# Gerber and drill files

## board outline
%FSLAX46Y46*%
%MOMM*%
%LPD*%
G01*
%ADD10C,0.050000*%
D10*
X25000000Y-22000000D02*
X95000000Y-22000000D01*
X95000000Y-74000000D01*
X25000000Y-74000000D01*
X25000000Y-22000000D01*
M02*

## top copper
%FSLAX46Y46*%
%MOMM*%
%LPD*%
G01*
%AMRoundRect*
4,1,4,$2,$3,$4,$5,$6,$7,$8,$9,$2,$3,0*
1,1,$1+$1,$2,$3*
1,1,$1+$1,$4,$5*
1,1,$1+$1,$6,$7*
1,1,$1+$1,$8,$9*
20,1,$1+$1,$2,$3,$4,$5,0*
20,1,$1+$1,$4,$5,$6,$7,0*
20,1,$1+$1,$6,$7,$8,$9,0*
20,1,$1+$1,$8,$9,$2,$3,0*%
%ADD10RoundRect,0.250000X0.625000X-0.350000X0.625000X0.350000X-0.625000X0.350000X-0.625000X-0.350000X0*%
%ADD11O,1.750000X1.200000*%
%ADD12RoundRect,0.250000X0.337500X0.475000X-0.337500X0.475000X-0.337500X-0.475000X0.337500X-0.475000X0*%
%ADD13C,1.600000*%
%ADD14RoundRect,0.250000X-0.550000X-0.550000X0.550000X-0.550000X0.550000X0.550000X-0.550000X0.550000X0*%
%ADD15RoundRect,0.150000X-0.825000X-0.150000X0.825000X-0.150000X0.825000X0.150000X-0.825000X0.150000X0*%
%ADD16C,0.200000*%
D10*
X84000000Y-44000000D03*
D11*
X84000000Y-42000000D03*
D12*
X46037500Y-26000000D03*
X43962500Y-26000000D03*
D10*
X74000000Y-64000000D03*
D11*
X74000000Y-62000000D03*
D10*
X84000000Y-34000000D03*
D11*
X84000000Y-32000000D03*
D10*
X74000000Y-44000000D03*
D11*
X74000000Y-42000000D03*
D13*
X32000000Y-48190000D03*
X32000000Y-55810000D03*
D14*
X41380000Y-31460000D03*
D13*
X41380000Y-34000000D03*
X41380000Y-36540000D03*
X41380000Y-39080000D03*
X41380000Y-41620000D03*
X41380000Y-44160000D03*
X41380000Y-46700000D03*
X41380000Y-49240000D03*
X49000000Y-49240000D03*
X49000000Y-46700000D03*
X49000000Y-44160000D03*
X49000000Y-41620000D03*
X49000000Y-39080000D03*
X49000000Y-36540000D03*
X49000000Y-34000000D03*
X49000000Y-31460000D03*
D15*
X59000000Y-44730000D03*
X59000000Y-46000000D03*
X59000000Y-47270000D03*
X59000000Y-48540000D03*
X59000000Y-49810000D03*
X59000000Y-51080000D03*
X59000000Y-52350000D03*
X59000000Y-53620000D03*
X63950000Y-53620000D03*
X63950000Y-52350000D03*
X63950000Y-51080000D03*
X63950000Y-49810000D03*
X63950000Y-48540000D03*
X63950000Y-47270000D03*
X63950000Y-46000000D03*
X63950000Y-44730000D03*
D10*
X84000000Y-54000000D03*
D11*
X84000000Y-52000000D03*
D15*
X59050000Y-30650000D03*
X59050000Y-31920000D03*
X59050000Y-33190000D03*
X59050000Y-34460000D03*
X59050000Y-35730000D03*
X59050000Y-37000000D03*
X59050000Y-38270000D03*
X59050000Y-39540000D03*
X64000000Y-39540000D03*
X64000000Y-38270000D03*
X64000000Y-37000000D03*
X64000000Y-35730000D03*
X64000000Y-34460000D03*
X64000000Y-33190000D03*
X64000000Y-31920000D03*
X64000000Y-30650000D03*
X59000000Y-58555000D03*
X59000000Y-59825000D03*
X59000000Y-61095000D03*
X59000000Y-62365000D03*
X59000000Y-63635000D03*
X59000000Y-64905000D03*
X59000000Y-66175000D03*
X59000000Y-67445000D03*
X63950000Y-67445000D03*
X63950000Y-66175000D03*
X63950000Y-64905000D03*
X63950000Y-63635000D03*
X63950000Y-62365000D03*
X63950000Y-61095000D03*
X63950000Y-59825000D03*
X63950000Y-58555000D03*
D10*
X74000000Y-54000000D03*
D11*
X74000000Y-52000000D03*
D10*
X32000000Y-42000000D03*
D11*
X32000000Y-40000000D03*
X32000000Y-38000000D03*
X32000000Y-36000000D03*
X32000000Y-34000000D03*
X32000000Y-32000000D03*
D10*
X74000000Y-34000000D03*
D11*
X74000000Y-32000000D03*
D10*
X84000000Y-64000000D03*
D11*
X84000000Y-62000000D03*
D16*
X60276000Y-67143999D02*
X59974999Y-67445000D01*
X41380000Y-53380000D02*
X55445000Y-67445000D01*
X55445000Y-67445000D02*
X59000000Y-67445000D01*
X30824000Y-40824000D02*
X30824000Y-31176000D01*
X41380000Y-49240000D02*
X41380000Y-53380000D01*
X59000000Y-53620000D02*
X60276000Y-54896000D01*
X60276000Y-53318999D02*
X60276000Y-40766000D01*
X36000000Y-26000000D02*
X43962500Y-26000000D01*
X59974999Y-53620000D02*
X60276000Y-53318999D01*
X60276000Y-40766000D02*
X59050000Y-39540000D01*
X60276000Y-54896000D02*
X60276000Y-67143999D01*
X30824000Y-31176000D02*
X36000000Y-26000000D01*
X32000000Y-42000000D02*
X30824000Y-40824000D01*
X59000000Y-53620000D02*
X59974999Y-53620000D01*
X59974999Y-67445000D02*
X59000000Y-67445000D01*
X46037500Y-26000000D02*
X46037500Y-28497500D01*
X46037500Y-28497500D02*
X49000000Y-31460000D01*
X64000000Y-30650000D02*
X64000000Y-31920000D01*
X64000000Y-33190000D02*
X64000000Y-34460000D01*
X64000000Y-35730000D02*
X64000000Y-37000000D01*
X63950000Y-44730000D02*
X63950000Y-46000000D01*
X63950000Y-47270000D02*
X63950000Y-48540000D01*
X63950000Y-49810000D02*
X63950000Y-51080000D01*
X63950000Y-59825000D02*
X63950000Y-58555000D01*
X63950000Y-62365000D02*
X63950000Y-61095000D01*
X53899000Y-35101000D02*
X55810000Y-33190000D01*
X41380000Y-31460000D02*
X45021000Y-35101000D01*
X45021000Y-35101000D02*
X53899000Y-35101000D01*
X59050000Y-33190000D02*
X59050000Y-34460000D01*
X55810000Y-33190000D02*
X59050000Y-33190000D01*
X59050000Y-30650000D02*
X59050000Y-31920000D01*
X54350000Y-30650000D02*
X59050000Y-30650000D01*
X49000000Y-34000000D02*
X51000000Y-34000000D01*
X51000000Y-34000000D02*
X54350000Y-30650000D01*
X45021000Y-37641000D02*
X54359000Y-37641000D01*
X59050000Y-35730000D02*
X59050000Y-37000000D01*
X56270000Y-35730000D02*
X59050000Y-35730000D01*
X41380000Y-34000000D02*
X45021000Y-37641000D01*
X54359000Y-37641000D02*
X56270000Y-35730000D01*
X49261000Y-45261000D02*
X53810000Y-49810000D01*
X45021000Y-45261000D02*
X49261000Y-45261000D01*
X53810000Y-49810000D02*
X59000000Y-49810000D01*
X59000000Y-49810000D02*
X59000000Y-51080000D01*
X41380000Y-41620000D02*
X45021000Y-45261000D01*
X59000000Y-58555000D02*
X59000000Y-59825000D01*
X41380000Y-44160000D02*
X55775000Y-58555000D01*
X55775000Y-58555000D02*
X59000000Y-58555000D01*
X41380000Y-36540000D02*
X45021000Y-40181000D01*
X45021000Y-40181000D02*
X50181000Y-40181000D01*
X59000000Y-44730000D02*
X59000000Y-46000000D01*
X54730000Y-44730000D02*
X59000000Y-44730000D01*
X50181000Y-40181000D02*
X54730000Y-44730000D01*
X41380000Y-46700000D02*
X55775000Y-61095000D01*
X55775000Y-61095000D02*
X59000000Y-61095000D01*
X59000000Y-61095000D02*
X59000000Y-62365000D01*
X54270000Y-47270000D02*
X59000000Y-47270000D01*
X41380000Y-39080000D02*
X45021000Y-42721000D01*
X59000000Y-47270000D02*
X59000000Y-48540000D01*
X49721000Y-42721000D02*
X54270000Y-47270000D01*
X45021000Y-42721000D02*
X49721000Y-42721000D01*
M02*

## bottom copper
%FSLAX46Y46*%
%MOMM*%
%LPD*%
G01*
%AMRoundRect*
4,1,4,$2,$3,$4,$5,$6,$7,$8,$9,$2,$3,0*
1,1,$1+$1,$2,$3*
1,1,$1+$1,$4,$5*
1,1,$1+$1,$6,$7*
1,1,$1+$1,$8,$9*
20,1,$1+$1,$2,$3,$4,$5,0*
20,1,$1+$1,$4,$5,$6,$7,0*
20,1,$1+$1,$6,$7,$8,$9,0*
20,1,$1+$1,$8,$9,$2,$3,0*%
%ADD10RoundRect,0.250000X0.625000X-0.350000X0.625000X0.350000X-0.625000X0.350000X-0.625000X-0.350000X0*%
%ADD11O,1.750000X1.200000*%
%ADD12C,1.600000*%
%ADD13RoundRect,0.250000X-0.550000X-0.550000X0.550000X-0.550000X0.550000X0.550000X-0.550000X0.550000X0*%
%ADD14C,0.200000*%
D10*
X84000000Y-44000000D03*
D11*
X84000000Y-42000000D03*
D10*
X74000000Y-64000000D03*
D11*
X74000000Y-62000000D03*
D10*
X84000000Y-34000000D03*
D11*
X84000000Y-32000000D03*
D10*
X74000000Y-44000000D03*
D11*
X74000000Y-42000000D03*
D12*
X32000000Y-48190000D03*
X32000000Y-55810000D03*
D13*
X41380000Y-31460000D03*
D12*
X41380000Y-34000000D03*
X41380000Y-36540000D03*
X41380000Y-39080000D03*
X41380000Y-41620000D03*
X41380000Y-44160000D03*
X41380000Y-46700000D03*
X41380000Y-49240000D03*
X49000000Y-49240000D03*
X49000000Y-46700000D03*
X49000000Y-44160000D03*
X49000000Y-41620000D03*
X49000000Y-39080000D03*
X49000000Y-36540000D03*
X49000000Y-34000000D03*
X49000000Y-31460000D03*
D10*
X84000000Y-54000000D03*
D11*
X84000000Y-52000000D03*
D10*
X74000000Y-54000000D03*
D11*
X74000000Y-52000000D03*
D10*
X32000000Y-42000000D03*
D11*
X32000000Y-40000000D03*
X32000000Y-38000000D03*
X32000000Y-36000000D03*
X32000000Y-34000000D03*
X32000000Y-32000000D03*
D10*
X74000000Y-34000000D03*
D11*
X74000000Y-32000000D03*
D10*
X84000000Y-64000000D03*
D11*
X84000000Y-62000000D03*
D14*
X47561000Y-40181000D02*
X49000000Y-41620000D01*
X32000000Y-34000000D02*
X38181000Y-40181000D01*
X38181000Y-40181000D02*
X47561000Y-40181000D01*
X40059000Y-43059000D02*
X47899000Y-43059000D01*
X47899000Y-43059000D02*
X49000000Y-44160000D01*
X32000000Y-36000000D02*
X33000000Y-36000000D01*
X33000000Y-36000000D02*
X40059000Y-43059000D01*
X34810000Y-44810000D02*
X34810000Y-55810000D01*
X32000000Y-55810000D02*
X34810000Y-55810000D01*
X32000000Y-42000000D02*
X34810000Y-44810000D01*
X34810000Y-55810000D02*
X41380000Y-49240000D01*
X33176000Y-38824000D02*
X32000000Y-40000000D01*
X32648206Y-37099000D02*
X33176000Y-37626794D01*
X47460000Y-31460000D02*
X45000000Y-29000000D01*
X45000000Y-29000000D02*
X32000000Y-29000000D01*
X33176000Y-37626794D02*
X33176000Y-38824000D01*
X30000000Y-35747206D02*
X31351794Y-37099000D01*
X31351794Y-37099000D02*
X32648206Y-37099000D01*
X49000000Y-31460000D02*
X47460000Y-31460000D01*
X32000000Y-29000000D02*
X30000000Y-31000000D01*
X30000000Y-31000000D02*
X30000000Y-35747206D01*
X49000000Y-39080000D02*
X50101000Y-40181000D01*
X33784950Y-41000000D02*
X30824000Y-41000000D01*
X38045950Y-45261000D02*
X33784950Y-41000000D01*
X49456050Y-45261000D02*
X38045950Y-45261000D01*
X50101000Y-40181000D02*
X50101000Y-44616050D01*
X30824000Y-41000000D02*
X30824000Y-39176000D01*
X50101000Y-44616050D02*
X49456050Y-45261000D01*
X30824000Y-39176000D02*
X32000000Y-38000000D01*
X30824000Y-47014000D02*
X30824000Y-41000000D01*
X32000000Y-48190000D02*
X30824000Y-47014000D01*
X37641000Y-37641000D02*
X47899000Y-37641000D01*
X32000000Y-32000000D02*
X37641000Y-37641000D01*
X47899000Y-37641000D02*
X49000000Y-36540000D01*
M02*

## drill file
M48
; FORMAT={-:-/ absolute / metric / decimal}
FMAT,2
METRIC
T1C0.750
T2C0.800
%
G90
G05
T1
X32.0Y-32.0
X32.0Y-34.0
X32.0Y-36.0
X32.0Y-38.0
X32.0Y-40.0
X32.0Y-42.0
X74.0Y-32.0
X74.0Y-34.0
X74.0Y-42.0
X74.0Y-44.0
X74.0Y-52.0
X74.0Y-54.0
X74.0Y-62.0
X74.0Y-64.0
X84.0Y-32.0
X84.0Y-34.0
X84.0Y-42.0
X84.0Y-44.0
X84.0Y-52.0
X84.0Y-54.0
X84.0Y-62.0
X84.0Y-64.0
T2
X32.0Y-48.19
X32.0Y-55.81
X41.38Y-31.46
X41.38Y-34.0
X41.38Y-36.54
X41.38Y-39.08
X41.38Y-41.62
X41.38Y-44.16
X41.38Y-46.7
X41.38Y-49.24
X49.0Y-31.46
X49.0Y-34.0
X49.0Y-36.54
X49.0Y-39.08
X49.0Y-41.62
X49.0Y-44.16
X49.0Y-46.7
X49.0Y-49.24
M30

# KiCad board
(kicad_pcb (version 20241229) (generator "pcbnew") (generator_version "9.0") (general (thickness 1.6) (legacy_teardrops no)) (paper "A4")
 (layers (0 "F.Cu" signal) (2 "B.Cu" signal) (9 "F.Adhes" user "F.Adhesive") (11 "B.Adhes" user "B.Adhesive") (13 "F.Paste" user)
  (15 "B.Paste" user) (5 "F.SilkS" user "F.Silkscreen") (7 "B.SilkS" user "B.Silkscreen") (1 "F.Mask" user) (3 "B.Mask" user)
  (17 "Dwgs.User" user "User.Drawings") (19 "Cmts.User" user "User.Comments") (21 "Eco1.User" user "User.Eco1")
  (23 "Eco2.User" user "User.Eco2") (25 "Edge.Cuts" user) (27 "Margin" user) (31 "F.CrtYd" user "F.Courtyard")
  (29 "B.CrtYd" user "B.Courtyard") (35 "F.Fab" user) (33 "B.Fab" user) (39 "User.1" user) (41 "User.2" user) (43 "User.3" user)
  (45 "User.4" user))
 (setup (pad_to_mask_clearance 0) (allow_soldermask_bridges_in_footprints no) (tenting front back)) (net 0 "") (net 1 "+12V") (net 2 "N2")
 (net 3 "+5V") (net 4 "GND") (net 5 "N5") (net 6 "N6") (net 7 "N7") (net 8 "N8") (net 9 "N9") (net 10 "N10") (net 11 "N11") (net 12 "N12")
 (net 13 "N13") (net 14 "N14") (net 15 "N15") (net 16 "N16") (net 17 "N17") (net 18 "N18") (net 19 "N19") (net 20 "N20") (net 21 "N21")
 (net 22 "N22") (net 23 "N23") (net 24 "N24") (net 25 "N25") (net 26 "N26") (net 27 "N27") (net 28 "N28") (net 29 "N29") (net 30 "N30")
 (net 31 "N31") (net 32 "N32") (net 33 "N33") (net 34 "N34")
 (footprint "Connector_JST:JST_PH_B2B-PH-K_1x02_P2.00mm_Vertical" (layer "F.Cu") (at 84 44 90)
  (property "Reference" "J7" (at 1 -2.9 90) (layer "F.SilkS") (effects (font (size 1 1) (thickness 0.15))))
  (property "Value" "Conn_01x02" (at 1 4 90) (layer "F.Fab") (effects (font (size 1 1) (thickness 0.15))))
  (pad "1" thru_hole roundrect (at 0 0 90) (size 1.2 1.75) (drill 0.75) (layers "*.Cu" "*.Mask") (remove_unused_layers no)
   (roundrect_rratio 0.208333) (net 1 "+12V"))
  (pad "2" thru_hole oval (at 2 0 90) (size 1.2 1.75) (drill 0.75) (layers "*.Cu" "*.Mask") (remove_unused_layers no) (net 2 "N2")))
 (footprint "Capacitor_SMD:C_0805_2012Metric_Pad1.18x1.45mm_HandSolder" (layer "F.Cu") (at 45 26 180)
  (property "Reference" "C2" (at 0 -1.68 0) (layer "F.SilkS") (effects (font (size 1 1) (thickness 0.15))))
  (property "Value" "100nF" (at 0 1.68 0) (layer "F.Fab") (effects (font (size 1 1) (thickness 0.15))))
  (pad "1" smd roundrect (at -1.0375 0 180) (size 1.175 1.45) (layers "F.Cu" "F.Mask" "F.Paste") (roundrect_rratio 0.212766) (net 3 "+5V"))
  (pad "2" smd roundrect (at 1.0375 0 180) (size 1.175 1.45) (layers "F.Cu" "F.Mask" "F.Paste") (roundrect_rratio 0.212766) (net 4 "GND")))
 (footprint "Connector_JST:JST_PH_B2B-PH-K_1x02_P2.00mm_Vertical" (layer "F.Cu") (at 74 64 90)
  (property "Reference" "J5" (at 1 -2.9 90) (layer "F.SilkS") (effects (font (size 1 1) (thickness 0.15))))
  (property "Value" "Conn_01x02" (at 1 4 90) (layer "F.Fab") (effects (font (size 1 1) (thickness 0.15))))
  (pad "1" thru_hole roundrect (at 0 0 90) (size 1.2 1.75) (drill 0.75) (layers "*.Cu" "*.Mask") (remove_unused_layers no)
   (roundrect_rratio 0.208333) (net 1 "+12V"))
  (pad "2" thru_hole oval (at 2 0 90) (size 1.2 1.75) (drill 0.75) (layers "*.Cu" "*.Mask") (remove_unused_layers no) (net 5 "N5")))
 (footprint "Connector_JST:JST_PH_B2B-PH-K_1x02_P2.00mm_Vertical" (layer "F.Cu") (at 84 34 90)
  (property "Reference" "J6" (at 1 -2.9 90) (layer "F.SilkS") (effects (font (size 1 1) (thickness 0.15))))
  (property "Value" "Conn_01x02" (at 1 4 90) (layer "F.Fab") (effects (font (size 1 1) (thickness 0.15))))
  (pad "1" thru_hole roundrect (at 0 0 90) (size 1.2 1.75) (drill 0.75) (layers "*.Cu" "*.Mask") (remove_unused_layers no)
   (roundrect_rratio 0.208333) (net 1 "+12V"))
  (pad "2" thru_hole oval (at 2 0 90) (size 1.2 1.75) (drill 0.75) (layers "*.Cu" "*.Mask") (remove_unused_layers no) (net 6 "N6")))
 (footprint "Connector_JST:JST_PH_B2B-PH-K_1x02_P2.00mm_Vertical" (layer "F.Cu") (at 74 44 90)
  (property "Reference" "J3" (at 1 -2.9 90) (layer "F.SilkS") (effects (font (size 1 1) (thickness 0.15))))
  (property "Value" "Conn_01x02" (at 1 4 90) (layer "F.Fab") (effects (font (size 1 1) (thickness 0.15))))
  (pad "1" thru_hole roundrect (at 0 0 90) (size 1.2 1.75) (drill 0.75) (layers "*.Cu" "*.Mask") (remove_unused_layers no)
   (roundrect_rratio 0.208333) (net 1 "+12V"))
  (pad "2" thru_hole oval (at 2 0 90) (size 1.2 1.75) (drill 0.75) (layers "*.Cu" "*.Mask") (remove_unused_layers no) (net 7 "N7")))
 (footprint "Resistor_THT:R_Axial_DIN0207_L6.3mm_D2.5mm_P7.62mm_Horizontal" (layer "F.Cu") (at 32 48.19 -90)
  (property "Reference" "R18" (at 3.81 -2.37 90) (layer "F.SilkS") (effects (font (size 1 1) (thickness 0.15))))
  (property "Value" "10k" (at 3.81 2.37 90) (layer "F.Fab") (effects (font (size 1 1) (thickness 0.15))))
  (pad "1" thru_hole circle (at 0 0 270) (size 1.6 1.6) (drill 0.8) (layers "*.Cu" "*.Mask") (remove_unused_layers no) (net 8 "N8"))
  (pad "2" thru_hole circle (at 7.62 0 270) (size 1.6 1.6) (drill 0.8) (layers "*.Cu" "*.Mask") (remove_unused_layers no) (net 4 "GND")))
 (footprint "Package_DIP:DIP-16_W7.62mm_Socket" (layer "F.Cu") (at 41.38 31.46)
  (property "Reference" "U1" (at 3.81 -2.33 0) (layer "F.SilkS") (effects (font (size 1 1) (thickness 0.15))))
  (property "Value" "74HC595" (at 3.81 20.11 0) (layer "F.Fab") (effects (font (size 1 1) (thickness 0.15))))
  (pad "1" thru_hole roundrect (at 0 0) (size 1.6 1.6) (drill 0.8) (layers "*.Cu" "*.Mask") (remove_unused_layers no)
   (roundrect_rratio 0.15625) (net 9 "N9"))
  (pad "2" thru_hole circle (at 0 2.54) (size 1.6 1.6) (drill 0.8) (layers "*.Cu" "*.Mask") (remove_unused_layers no) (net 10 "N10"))
  (pad "3" thru_hole circle (at 0 5.08) (size 1.6 1.6) (drill 0.8) (layers "*.Cu" "*.Mask") (remove_unused_layers no) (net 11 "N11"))
  (pad "4" thru_hole circle (at 0 7.62) (size 1.6 1.6) (drill 0.8) (layers "*.Cu" "*.Mask") (remove_unused_layers no) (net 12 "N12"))
  (pad "5" thru_hole circle (at 0 10.16) (size 1.6 1.6) (drill 0.8) (layers "*.Cu" "*.Mask") (remove_unused_layers no) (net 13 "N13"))
  (pad "6" thru_hole circle (at 0 12.7) (size 1.6 1.6) (drill 0.8) (layers "*.Cu" "*.Mask") (remove_unused_layers no) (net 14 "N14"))
  (pad "7" thru_hole circle (at 0 15.24) (size 1.6 1.6) (drill 0.8) (layers "*.Cu" "*.Mask") (remove_unused_layers no) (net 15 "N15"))
  (pad "8" thru_hole circle (at 0 17.78) (size 1.6 1.6) (drill 0.8) (layers "*.Cu" "*.Mask") (remove_unused_layers no) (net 4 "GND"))
  (pad "9" thru_hole circle (at 7.62 17.78) (size 1.6 1.6) (drill 0.8) (layers "*.Cu" "*.Mask") (remove_unused_layers no) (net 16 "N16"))
  (pad "10" thru_hole circle (at 7.62 15.24) (size 1.6 1.6) (drill 0.8) (layers "*.Cu" "*.Mask") (remove_unused_layers no) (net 3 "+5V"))
  (pad "11" thru_hole circle (at 7.62 12.7) (size 1.6 1.6) (drill 0.8) (layers "*.Cu" "*.Mask") (remove_unused_layers no) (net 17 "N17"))
  (pad "12" thru_hole circle (at 7.62 10.16) (size 1.6 1.6) (drill 0.8) (layers "*.Cu" "*.Mask") (remove_unused_layers no) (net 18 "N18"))
  (pad "13" thru_hole circle (at 7.62 7.62) (size 1.6 1.6) (drill 0.8) (layers "*.Cu" "*.Mask") (remove_unused_layers no) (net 8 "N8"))
  (pad "14" thru_hole circle (at 7.62 5.08) (size 1.6 1.6) (drill 0.8) (layers "*.Cu" "*.Mask") (remove_unused_layers no) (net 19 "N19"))
  (pad "15" thru_hole circle (at 7.62 2.54) (size 1.6 1.6) (drill 0.8) (layers "*.Cu" "*.Mask") (remove_unused_layers no) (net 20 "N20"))
  (pad "16" thru_hole circle (at 7.62 0) (size 1.6 1.6) (drill 0.8) (layers "*.Cu" "*.Mask") (remove_unused_layers no) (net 3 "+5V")))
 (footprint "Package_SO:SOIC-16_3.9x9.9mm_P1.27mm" (layer "F.Cu") (at 61.475 49.175)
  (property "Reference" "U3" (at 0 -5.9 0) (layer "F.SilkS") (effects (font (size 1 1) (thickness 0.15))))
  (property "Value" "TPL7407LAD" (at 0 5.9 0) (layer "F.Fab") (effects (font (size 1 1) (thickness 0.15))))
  (pad "1" smd roundrect (at -2.475 -4.445) (size 1.95 0.6) (layers "F.Cu" "F.Mask" "F.Paste") (roundrect_rratio 0.25) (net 11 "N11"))
  (pad "2" smd roundrect (at -2.475 -3.175) (size 1.95 0.6) (layers "F.Cu" "F.Mask" "F.Paste") (roundrect_rratio 0.25) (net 11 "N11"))
  (pad "3" smd roundrect (at -2.475 -1.905) (size 1.95 0.6) (layers "F.Cu" "F.Mask" "F.Paste") (roundrect_rratio 0.25) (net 12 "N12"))
  (pad "4" smd roundrect (at -2.475 -0.635) (size 1.95 0.6) (layers "F.Cu" "F.Mask" "F.Paste") (roundrect_rratio 0.25) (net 12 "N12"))
  (pad "5" smd roundrect (at -2.475 0.635) (size 1.95 0.6) (layers "F.Cu" "F.Mask" "F.Paste") (roundrect_rratio 0.25) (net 13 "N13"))
  (pad "6" smd roundrect (at -2.475 1.905) (size 1.95 0.6) (layers "F.Cu" "F.Mask" "F.Paste") (roundrect_rratio 0.25) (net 13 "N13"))
  (pad "7" smd roundrect (at -2.475 3.175) (size 1.95 0.6) (layers "F.Cu" "F.Mask" "F.Paste") (roundrect_rratio 0.25) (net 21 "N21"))
  (pad "8" smd roundrect (at -2.475 4.445) (size 1.95 0.6) (layers "F.Cu" "F.Mask" "F.Paste") (roundrect_rratio 0.25) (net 4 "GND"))
  (pad "9" smd roundrect (at 2.475 4.445) (size 1.95 0.6) (layers "F.Cu" "F.Mask" "F.Paste") (roundrect_rratio 0.25) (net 1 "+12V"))
  (pad "10" smd roundrect (at 2.475 3.175) (size 1.95 0.6) (layers "F.Cu" "F.Mask" "F.Paste") (roundrect_rratio 0.25) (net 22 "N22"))
  (pad "11" smd roundrect (at 2.475 1.905) (size 1.95 0.6) (layers "F.Cu" "F.Mask" "F.Paste") (roundrect_rratio 0.25) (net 2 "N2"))
  (pad "12" smd roundrect (at 2.475 0.635) (size 1.95 0.6) (layers "F.Cu" "F.Mask" "F.Paste") (roundrect_rratio 0.25) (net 2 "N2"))
  (pad "13" smd roundrect (at 2.475 -0.635) (size 1.95 0.6) (layers "F.Cu" "F.Mask" "F.Paste") (roundrect_rratio 0.25) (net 6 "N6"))
  (pad "14" smd roundrect (at 2.475 -1.905) (size 1.95 0.6) (layers "F.Cu" "F.Mask" "F.Paste") (roundrect_rratio 0.25) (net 6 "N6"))
  (pad "15" smd roundrect (at 2.475 -3.175) (size 1.95 0.6) (layers "F.Cu" "F.Mask" "F.Paste") (roundrect_rratio 0.25) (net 5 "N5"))
  (pad "16" smd roundrect (at 2.475 -4.445) (size 1.95 0.6) (layers "F.Cu" "F.Mask" "F.Paste") (roundrect_rratio 0.25) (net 5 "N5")))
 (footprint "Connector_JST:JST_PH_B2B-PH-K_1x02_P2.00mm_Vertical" (layer "F.Cu") (at 84 54 90)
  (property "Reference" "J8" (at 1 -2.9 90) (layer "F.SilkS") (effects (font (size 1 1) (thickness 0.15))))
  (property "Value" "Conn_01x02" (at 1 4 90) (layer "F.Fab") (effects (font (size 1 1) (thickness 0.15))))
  (pad "1" thru_hole roundrect (at 0 0 90) (size 1.2 1.75) (drill 0.75) (layers "*.Cu" "*.Mask") (remove_unused_layers no)
   (roundrect_rratio 0.208333) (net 1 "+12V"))
  (pad "2" thru_hole oval (at 2 0 90) (size 1.2 1.75) (drill 0.75) (layers "*.Cu" "*.Mask") (remove_unused_layers no) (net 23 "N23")))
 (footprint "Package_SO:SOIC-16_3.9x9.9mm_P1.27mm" (layer "F.Cu") (at 61.525 35.095)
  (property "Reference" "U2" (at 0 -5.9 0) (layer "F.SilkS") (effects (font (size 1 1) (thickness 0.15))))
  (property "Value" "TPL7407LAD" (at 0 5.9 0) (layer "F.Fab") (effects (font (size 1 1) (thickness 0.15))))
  (pad "1" smd roundrect (at -2.475 -4.445) (size 1.95 0.6) (layers "F.Cu" "F.Mask" "F.Paste") (roundrect_rratio 0.25) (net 20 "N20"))
  (pad "2" smd roundrect (at -2.475 -3.175) (size 1.95 0.6) (layers "F.Cu" "F.Mask" "F.Paste") (roundrect_rratio 0.25) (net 20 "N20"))
  (pad "3" smd roundrect (at -2.475 -1.905) (size 1.95 0.6) (layers "F.Cu" "F.Mask" "F.Paste") (roundrect_rratio 0.25) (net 9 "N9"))
  (pad "4" smd roundrect (at -2.475 -0.635) (size 1.95 0.6) (layers "F.Cu" "F.Mask" "F.Paste") (roundrect_rratio 0.25) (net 9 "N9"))
  (pad "5" smd roundrect (at -2.475 0.635) (size 1.95 0.6) (layers "F.Cu" "F.Mask" "F.Paste") (roundrect_rratio 0.25) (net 10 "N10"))
  (pad "6" smd roundrect (at -2.475 1.905) (size 1.95 0.6) (layers "F.Cu" "F.Mask" "F.Paste") (roundrect_rratio 0.25) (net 10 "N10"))
  (pad "7" smd roundrect (at -2.475 3.175) (size 1.95 0.6) (layers "F.Cu" "F.Mask" "F.Paste") (roundrect_rratio 0.25) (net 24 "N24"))
  (pad "8" smd roundrect (at -2.475 4.445) (size 1.95 0.6) (layers "F.Cu" "F.Mask" "F.Paste") (roundrect_rratio 0.25) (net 4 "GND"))
  (pad "9" smd roundrect (at 2.475 4.445) (size 1.95 0.6) (layers "F.Cu" "F.Mask" "F.Paste") (roundrect_rratio 0.25) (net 1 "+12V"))
  (pad "10" smd roundrect (at 2.475 3.175) (size 1.95 0.6) (layers "F.Cu" "F.Mask" "F.Paste") (roundrect_rratio 0.25) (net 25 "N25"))
  (pad "11" smd roundrect (at 2.475 1.905) (size 1.95 0.6) (layers "F.Cu" "F.Mask" "F.Paste") (roundrect_rratio 0.25) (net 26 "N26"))
  (pad "12" smd roundrect (at 2.475 0.635) (size 1.95 0.6) (layers "F.Cu" "F.Mask" "F.Paste") (roundrect_rratio 0.25) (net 26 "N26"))
  (pad "13" smd roundrect (at 2.475 -0.635) (size 1.95 0.6) (layers "F.Cu" "F.Mask" "F.Paste") (roundrect_rratio 0.25) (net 7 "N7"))
  (pad "14" smd roundrect (at 2.475 -1.905) (size 1.95 0.6) (layers "F.Cu" "F.Mask" "F.Paste") (roundrect_rratio 0.25) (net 7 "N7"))
  (pad "15" smd roundrect (at 2.475 -3.175) (size 1.95 0.6) (layers "F.Cu" "F.Mask" "F.Paste") (roundrect_rratio 0.25) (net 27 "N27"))
  (pad "16" smd roundrect (at 2.475 -4.445) (size 1.95 0.6) (layers "F.Cu" "F.Mask" "F.Paste") (roundrect_rratio 0.25) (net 27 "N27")))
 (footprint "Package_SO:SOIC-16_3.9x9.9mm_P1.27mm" (layer "F.Cu") (at 61.475 63)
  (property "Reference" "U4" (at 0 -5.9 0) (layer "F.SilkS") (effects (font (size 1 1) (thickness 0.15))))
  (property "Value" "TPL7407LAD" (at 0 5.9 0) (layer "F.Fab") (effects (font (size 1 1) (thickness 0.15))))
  (pad "1" smd roundrect (at -2.475 -4.445) (size 1.95 0.6) (layers "F.Cu" "F.Mask" "F.Paste") (roundrect_rratio 0.25) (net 14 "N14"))
  (pad "2" smd roundrect (at -2.475 -3.175) (size 1.95 0.6) (layers "F.Cu" "F.Mask" "F.Paste") (roundrect_rratio 0.25) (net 14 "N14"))
  (pad "3" smd roundrect (at -2.475 -1.905) (size 1.95 0.6) (layers "F.Cu" "F.Mask" "F.Paste") (roundrect_rratio 0.25) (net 15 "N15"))
  (pad "4" smd roundrect (at -2.475 -0.635) (size 1.95 0.6) (layers "F.Cu" "F.Mask" "F.Paste") (roundrect_rratio 0.25) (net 15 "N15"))
  (pad "5" smd roundrect (at -2.475 0.635) (size 1.95 0.6) (layers "F.Cu" "F.Mask" "F.Paste") (roundrect_rratio 0.25) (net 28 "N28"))
  (pad "6" smd roundrect (at -2.475 1.905) (size 1.95 0.6) (layers "F.Cu" "F.Mask" "F.Paste") (roundrect_rratio 0.25) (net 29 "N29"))
  (pad "7" smd roundrect (at -2.475 3.175) (size 1.95 0.6) (layers "F.Cu" "F.Mask" "F.Paste") (roundrect_rratio 0.25) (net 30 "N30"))
  (pad "8" smd roundrect (at -2.475 4.445) (size 1.95 0.6) (layers "F.Cu" "F.Mask" "F.Paste") (roundrect_rratio 0.25) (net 4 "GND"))
  (pad "9" smd roundrect (at 2.475 4.445) (size 1.95 0.6) (layers "F.Cu" "F.Mask" "F.Paste") (roundrect_rratio 0.25) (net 1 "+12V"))
  (pad "10" smd roundrect (at 2.475 3.175) (size 1.95 0.6) (layers "F.Cu" "F.Mask" "F.Paste") (roundrect_rratio 0.25) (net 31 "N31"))
  (pad "11" smd roundrect (at 2.475 1.905) (size 1.95 0.6) (layers "F.Cu" "F.Mask" "F.Paste") (roundrect_rratio 0.25) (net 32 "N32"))
  (pad "12" smd roundrect (at 2.475 0.635) (size 1.95 0.6) (layers "F.Cu" "F.Mask" "F.Paste") (roundrect_rratio 0.25) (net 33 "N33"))
  (pad "13" smd roundrect (at 2.475 -0.635) (size 1.95 0.6) (layers "F.Cu" "F.Mask" "F.Paste") (roundrect_rratio 0.25) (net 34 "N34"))
  (pad "14" smd roundrect (at 2.475 -1.905) (size 1.95 0.6) (layers "F.Cu" "F.Mask" "F.Paste") (roundrect_rratio 0.25) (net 34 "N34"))
  (pad "15" smd roundrect (at 2.475 -3.175) (size 1.95 0.6) (layers "F.Cu" "F.Mask" "F.Paste") (roundrect_rratio 0.25) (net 23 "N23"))
  (pad "16" smd roundrect (at 2.475 -4.445) (size 1.95 0.6) (layers "F.Cu" "F.Mask" "F.Paste") (roundrect_rratio 0.25) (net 23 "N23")))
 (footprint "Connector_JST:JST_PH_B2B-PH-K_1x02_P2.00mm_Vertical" (layer "F.Cu") (at 74 54 90)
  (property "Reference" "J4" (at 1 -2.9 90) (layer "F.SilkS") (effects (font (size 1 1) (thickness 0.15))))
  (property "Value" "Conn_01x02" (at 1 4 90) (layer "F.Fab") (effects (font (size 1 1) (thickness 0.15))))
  (pad "1" thru_hole roundrect (at 0 0 90) (size 1.2 1.75) (drill 0.75) (layers "*.Cu" "*.Mask") (remove_unused_layers no)
   (roundrect_rratio 0.208333) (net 1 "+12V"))
  (pad "2" thru_hole oval (at 2 0 90) (size 1.2 1.75) (drill 0.75) (layers "*.Cu" "*.Mask") (remove_unused_layers no) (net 26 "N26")))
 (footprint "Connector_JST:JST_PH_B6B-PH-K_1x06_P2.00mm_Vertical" (layer "F.Cu") (at 32 42 90)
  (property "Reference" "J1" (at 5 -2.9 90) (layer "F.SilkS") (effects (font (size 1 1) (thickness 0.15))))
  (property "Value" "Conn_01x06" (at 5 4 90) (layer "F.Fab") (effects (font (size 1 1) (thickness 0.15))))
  (pad "1" thru_hole roundrect (at 0 0 90) (size 1.2 1.75) (drill 0.75) (layers "*.Cu" "*.Mask") (remove_unused_layers no)
   (roundrect_rratio 0.208333) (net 4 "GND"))
  (pad "2" thru_hole oval (at 2 0 90) (size 1.2 1.75) (drill 0.75) (layers "*.Cu" "*.Mask") (remove_unused_layers no) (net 3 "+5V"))
  (pad "3" thru_hole oval (at 4 0 90) (size 1.2 1.75) (drill 0.75) (layers "*.Cu" "*.Mask") (remove_unused_layers no) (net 8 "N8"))
  (pad "4" thru_hole oval (at 6 0 90) (size 1.2 1.75) (drill 0.75) (layers "*.Cu" "*.Mask") (remove_unused_layers no) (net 17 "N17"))
  (pad "5" thru_hole oval (at 8 0 90) (size 1.2 1.75) (drill 0.75) (layers "*.Cu" "*.Mask") (remove_unused_layers no) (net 18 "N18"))
  (pad "6" thru_hole oval (at 10 0 90) (size 1.2 1.75) (drill 0.75) (layers "*.Cu" "*.Mask") (remove_unused_layers no) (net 19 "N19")))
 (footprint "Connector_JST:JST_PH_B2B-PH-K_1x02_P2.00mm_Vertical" (layer "F.Cu") (at 74 34 90)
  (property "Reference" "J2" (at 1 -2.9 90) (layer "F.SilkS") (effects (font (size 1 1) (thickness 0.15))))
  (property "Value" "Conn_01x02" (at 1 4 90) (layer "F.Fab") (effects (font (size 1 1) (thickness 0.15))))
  (pad "1" thru_hole roundrect (at 0 0 90) (size 1.2 1.75) (drill 0.75) (layers "*.Cu" "*.Mask") (remove_unused_layers no)
   (roundrect_rratio 0.208333) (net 1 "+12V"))
  (pad "2" thru_hole oval (at 2 0 90) (size 1.2 1.75) (drill 0.75) (layers "*.Cu" "*.Mask") (remove_unused_layers no) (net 27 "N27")))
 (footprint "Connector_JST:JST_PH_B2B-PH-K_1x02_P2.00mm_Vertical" (layer "F.Cu") (at 84 64 90)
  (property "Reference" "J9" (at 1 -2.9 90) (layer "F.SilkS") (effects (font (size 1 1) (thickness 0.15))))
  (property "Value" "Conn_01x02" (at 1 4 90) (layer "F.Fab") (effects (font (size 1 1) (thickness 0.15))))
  (pad "1" thru_hole roundrect (at 0 0 90) (size 1.2 1.75) (drill 0.75) (layers "*.Cu" "*.Mask") (remove_unused_layers no)
   (roundrect_rratio 0.208333) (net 1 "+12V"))
  (pad "2" thru_hole oval (at 2 0 90) (size 1.2 1.75) (drill 0.75) (layers "*.Cu" "*.Mask") (remove_unused_layers no) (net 34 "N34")))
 (gr_rect (start 25 22) (end 95 74) (stroke (width 0.05) (type default)) (fill no) (layer "Edge.Cuts"))
 (segment (start 47.561 40.181) (end 49 41.62) (width 0.2) (layer "B.Cu") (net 18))
 (segment (start 32 34) (end 38.181 40.181) (width 0.2) (layer "B.Cu") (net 18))
 (segment (start 38.181 40.181) (end 47.561 40.181) (width 0.2) (layer "B.Cu") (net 18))
 (segment (start 40.059 43.059) (end 47.899 43.059) (width 0.2) (layer "B.Cu") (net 17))
 (segment (start 47.899 43.059) (end 49 44.16) (width 0.2) (layer "B.Cu") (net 17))
 (segment (start 32 36) (end 33 36) (width 0.2) (layer "B.Cu") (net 17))
 (segment (start 33 36) (end 40.059 43.059) (width 0.2) (layer "B.Cu") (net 17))
 (segment (start 60.276 67.143999) (end 59.974999 67.445) (width 0.2) (layer "F.Cu") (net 4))
 (segment (start 41.38 53.38) (end 55.445 67.445) (width 0.2) (layer "F.Cu") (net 4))
 (segment (start 55.445 67.445) (end 59 67.445) (width 0.2) (layer "F.Cu") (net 4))
 (segment (start 30.824 40.824) (end 30.824 31.176) (width 0.2) (layer "F.Cu") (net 4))
 (segment (start 41.38 49.24) (end 41.38 53.38) (width 0.2) (layer "F.Cu") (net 4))
 (segment (start 59 53.62) (end 60.276 54.896) (width 0.2) (layer "F.Cu") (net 4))
 (segment (start 60.276 53.318999) (end 60.276 40.766) (width 0.2) (layer "F.Cu") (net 4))
 (segment (start 36 26) (end 43.9625 26) (width 0.2) (layer "F.Cu") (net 4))
 (segment (start 59.974999 53.62) (end 60.276 53.318999) (width 0.2) (layer "F.Cu") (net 4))
 (segment (start 60.276 40.766) (end 59.05 39.54) (width 0.2) (layer "F.Cu") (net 4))
 (segment (start 60.276 54.896) (end 60.276 67.143999) (width 0.2) (layer "F.Cu") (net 4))
 (segment (start 30.824 31.176) (end 36 26) (width 0.2) (layer "F.Cu") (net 4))
 (segment (start 32 42) (end 30.824 40.824) (width 0.2) (layer "F.Cu") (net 4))
 (segment (start 59 53.62) (end 59.974999 53.62) (width 0.2) (layer "F.Cu") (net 4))
 (segment (start 59.974999 67.445) (end 59 67.445) (width 0.2) (layer "F.Cu") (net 4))
 (segment (start 34.81 44.81) (end 34.81 55.81) (width 0.2) (layer "B.Cu") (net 4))
 (segment (start 32 55.81) (end 34.81 55.81) (width 0.2) (layer "B.Cu") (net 4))
 (segment (start 32 42) (end 34.81 44.81) (width 0.2) (layer "B.Cu") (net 4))
 (segment (start 34.81 55.81) (end 41.38 49.24) (width 0.2) (layer "B.Cu") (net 4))
 (segment (start 46.0375 26) (end 46.0375 28.4975) (width 0.2) (layer "F.Cu") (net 3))
 (segment (start 46.0375 28.4975) (end 49 31.46) (width 0.2) (layer "F.Cu") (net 3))
 (segment (start 33.176 38.824) (end 32 40) (width 0.2) (layer "B.Cu") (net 3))
 (segment (start 32.648206 37.099) (end 33.176 37.626794) (width 0.2) (layer "B.Cu") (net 3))
 (segment (start 47.46 31.46) (end 45 29) (width 0.2) (layer "B.Cu") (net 3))
 (segment (start 45 29) (end 32 29) (width 0.2) (layer "B.Cu") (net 3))
 (segment (start 33.176 37.626794) (end 33.176 38.824) (width 0.2) (layer "B.Cu") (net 3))
 (segment (start 30 35.747206) (end 31.351794 37.099) (width 0.2) (layer "B.Cu") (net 3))
 (segment (start 31.351794 37.099) (end 32.648206 37.099) (width 0.2) (layer "B.Cu") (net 3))
 (segment (start 49 31.46) (end 47.46 31.46) (width 0.2) (layer "B.Cu") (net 3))
 (segment (start 32 29) (end 30 31) (width 0.2) (layer "B.Cu") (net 3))
 (segment (start 30 31) (end 30 35.747206) (width 0.2) (layer "B.Cu") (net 3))
 (segment (start 49 39.08) (end 50.101 40.181) (width 0.2) (layer "B.Cu") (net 8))
 (segment (start 33.78495 41) (end 30.824 41) (width 0.2) (layer "B.Cu") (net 8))
 (segment (start 38.04595 45.261) (end 33.78495 41) (width 0.2) (layer "B.Cu") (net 8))
 (segment (start 49.45605 45.261) (end 38.04595 45.261) (width 0.2) (layer "B.Cu") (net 8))
 (segment (start 50.101 40.181) (end 50.101 44.61605) (width 0.2) (layer "B.Cu") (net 8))
 (segment (start 30.824 41) (end 30.824 39.176) (width 0.2) (layer "B.Cu") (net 8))
 (segment (start 50.101 44.61605) (end 49.45605 45.261) (width 0.2) (layer "B.Cu") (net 8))
 (segment (start 30.824 39.176) (end 32 38) (width 0.2) (layer "B.Cu") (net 8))
 (segment (start 30.824 47.014) (end 30.824 41) (width 0.2) (layer "B.Cu") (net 8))
 (segment (start 32 48.19) (end 30.824 47.014) (width 0.2) (layer "B.Cu") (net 8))
 (segment (start 37.641 37.641) (end 47.899 37.641) (width 0.2) (layer "B.Cu") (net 19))
 (segment (start 32 32) (end 37.641 37.641) (width 0.2) (layer "B.Cu") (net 19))
 (segment (start 47.899 37.641) (end 49 36.54) (width 0.2) (layer "B.Cu") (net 19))
 (segment (start 64 30.65) (end 64 31.92) (width 0.2) (layer "F.Cu") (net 27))
 (segment (start 64 33.19) (end 64 34.46) (width 0.2) (layer "F.Cu") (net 7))
 (segment (start 64 35.73) (end 64 37) (width 0.2) (layer "F.Cu") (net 26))
 (segment (start 63.95 44.73) (end 63.95 46) (width 0.2) (layer "F.Cu") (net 5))
 (segment (start 63.95 47.27) (end 63.95 48.54) (width 0.2) (layer "F.Cu") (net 6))
 (segment (start 63.95 49.81) (end 63.95 51.08) (width 0.2) (layer "F.Cu") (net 2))
 (segment (start 63.95 59.825) (end 63.95 58.555) (width 0.2) (layer "F.Cu") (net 23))
 (segment (start 63.95 62.365) (end 63.95 61.095) (width 0.2) (layer "F.Cu") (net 34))
 (segment (start 53.899 35.101) (end 55.81 33.19) (width 0.2) (layer "F.Cu") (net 9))
 (segment (start 41.38 31.46) (end 45.021 35.101) (width 0.2) (layer "F.Cu") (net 9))
 (segment (start 45.021 35.101) (end 53.899 35.101) (width 0.2) (layer "F.Cu") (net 9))
 (segment (start 59.05 33.19) (end 59.05 34.46) (width 0.2) (layer "F.Cu") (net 9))
 (segment (start 55.81 33.19) (end 59.05 33.19) (width 0.2) (layer "F.Cu") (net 9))
 (segment (start 59.05 30.65) (end 59.05 31.92) (width 0.2) (layer "F.Cu") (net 20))
 (segment (start 54.35 30.65) (end 59.05 30.65) (width 0.2) (layer "F.Cu") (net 20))
 (segment (start 49 34) (end 51 34) (width 0.2) (layer "F.Cu") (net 20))
 (segment (start 51 34) (end 54.35 30.65) (width 0.2) (layer "F.Cu") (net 20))
 (segment (start 45.021 37.641) (end 54.359 37.641) (width 0.2) (layer "F.Cu") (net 10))
 (segment (start 59.05 35.73) (end 59.05 37) (width 0.2) (layer "F.Cu") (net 10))
 (segment (start 56.27 35.73) (end 59.05 35.73) (width 0.2) (layer "F.Cu") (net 10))
 (segment (start 41.38 34) (end 45.021 37.641) (width 0.2) (layer "F.Cu") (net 10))
 (segment (start 54.359 37.641) (end 56.27 35.73) (width 0.2) (layer "F.Cu") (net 10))
 (segment (start 49.261 45.261) (end 53.81 49.81) (width 0.2) (layer "F.Cu") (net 13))
 (segment (start 45.021 45.261) (end 49.261 45.261) (width 0.2) (layer "F.Cu") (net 13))
 (segment (start 53.81 49.81) (end 59 49.81) (width 0.2) (layer "F.Cu") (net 13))
 (segment (start 59 49.81) (end 59 51.08) (width 0.2) (layer "F.Cu") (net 13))
 (segment (start 41.38 41.62) (end 45.021 45.261) (width 0.2) (layer "F.Cu") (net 13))
 (segment (start 59 58.555) (end 59 59.825) (width 0.2) (layer "F.Cu") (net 14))
 (segment (start 41.38 44.16) (end 55.775 58.555) (width 0.2) (layer "F.Cu") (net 14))
 (segment (start 55.775 58.555) (end 59 58.555) (width 0.2) (layer "F.Cu") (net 14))
 (segment (start 41.38 36.54) (end 45.021 40.181) (width 0.2) (layer "F.Cu") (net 11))
 (segment (start 45.021 40.181) (end 50.181 40.181) (width 0.2) (layer "F.Cu") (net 11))
 (segment (start 59 44.73) (end 59 46) (width 0.2) (layer "F.Cu") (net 11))
 (segment (start 54.73 44.73) (end 59 44.73) (width 0.2) (layer "F.Cu") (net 11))
 (segment (start 50.181 40.181) (end 54.73 44.73) (width 0.2) (layer "F.Cu") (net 11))
 (segment (start 41.38 46.7) (end 55.775 61.095) (width 0.2) (layer "F.Cu") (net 15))
 (segment (start 55.775 61.095) (end 59 61.095) (width 0.2) (layer "F.Cu") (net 15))
 (segment (start 59 61.095) (end 59 62.365) (width 0.2) (layer "F.Cu") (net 15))
 (segment (start 54.27 47.27) (end 59 47.27) (width 0.2) (layer "F.Cu") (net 12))
 (segment (start 41.38 39.08) (end 45.021 42.721) (width 0.2) (layer "F.Cu") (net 12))
 (segment (start 59 47.27) (end 59 48.54) (width 0.2) (layer "F.Cu") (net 12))
 (segment (start 49.721 42.721) (end 54.27 47.27) (width 0.2) (layer "F.Cu") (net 12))
 (segment (start 45.021 42.721) (end 49.721 42.721) (width 0.2) (layer "F.Cu") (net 12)))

